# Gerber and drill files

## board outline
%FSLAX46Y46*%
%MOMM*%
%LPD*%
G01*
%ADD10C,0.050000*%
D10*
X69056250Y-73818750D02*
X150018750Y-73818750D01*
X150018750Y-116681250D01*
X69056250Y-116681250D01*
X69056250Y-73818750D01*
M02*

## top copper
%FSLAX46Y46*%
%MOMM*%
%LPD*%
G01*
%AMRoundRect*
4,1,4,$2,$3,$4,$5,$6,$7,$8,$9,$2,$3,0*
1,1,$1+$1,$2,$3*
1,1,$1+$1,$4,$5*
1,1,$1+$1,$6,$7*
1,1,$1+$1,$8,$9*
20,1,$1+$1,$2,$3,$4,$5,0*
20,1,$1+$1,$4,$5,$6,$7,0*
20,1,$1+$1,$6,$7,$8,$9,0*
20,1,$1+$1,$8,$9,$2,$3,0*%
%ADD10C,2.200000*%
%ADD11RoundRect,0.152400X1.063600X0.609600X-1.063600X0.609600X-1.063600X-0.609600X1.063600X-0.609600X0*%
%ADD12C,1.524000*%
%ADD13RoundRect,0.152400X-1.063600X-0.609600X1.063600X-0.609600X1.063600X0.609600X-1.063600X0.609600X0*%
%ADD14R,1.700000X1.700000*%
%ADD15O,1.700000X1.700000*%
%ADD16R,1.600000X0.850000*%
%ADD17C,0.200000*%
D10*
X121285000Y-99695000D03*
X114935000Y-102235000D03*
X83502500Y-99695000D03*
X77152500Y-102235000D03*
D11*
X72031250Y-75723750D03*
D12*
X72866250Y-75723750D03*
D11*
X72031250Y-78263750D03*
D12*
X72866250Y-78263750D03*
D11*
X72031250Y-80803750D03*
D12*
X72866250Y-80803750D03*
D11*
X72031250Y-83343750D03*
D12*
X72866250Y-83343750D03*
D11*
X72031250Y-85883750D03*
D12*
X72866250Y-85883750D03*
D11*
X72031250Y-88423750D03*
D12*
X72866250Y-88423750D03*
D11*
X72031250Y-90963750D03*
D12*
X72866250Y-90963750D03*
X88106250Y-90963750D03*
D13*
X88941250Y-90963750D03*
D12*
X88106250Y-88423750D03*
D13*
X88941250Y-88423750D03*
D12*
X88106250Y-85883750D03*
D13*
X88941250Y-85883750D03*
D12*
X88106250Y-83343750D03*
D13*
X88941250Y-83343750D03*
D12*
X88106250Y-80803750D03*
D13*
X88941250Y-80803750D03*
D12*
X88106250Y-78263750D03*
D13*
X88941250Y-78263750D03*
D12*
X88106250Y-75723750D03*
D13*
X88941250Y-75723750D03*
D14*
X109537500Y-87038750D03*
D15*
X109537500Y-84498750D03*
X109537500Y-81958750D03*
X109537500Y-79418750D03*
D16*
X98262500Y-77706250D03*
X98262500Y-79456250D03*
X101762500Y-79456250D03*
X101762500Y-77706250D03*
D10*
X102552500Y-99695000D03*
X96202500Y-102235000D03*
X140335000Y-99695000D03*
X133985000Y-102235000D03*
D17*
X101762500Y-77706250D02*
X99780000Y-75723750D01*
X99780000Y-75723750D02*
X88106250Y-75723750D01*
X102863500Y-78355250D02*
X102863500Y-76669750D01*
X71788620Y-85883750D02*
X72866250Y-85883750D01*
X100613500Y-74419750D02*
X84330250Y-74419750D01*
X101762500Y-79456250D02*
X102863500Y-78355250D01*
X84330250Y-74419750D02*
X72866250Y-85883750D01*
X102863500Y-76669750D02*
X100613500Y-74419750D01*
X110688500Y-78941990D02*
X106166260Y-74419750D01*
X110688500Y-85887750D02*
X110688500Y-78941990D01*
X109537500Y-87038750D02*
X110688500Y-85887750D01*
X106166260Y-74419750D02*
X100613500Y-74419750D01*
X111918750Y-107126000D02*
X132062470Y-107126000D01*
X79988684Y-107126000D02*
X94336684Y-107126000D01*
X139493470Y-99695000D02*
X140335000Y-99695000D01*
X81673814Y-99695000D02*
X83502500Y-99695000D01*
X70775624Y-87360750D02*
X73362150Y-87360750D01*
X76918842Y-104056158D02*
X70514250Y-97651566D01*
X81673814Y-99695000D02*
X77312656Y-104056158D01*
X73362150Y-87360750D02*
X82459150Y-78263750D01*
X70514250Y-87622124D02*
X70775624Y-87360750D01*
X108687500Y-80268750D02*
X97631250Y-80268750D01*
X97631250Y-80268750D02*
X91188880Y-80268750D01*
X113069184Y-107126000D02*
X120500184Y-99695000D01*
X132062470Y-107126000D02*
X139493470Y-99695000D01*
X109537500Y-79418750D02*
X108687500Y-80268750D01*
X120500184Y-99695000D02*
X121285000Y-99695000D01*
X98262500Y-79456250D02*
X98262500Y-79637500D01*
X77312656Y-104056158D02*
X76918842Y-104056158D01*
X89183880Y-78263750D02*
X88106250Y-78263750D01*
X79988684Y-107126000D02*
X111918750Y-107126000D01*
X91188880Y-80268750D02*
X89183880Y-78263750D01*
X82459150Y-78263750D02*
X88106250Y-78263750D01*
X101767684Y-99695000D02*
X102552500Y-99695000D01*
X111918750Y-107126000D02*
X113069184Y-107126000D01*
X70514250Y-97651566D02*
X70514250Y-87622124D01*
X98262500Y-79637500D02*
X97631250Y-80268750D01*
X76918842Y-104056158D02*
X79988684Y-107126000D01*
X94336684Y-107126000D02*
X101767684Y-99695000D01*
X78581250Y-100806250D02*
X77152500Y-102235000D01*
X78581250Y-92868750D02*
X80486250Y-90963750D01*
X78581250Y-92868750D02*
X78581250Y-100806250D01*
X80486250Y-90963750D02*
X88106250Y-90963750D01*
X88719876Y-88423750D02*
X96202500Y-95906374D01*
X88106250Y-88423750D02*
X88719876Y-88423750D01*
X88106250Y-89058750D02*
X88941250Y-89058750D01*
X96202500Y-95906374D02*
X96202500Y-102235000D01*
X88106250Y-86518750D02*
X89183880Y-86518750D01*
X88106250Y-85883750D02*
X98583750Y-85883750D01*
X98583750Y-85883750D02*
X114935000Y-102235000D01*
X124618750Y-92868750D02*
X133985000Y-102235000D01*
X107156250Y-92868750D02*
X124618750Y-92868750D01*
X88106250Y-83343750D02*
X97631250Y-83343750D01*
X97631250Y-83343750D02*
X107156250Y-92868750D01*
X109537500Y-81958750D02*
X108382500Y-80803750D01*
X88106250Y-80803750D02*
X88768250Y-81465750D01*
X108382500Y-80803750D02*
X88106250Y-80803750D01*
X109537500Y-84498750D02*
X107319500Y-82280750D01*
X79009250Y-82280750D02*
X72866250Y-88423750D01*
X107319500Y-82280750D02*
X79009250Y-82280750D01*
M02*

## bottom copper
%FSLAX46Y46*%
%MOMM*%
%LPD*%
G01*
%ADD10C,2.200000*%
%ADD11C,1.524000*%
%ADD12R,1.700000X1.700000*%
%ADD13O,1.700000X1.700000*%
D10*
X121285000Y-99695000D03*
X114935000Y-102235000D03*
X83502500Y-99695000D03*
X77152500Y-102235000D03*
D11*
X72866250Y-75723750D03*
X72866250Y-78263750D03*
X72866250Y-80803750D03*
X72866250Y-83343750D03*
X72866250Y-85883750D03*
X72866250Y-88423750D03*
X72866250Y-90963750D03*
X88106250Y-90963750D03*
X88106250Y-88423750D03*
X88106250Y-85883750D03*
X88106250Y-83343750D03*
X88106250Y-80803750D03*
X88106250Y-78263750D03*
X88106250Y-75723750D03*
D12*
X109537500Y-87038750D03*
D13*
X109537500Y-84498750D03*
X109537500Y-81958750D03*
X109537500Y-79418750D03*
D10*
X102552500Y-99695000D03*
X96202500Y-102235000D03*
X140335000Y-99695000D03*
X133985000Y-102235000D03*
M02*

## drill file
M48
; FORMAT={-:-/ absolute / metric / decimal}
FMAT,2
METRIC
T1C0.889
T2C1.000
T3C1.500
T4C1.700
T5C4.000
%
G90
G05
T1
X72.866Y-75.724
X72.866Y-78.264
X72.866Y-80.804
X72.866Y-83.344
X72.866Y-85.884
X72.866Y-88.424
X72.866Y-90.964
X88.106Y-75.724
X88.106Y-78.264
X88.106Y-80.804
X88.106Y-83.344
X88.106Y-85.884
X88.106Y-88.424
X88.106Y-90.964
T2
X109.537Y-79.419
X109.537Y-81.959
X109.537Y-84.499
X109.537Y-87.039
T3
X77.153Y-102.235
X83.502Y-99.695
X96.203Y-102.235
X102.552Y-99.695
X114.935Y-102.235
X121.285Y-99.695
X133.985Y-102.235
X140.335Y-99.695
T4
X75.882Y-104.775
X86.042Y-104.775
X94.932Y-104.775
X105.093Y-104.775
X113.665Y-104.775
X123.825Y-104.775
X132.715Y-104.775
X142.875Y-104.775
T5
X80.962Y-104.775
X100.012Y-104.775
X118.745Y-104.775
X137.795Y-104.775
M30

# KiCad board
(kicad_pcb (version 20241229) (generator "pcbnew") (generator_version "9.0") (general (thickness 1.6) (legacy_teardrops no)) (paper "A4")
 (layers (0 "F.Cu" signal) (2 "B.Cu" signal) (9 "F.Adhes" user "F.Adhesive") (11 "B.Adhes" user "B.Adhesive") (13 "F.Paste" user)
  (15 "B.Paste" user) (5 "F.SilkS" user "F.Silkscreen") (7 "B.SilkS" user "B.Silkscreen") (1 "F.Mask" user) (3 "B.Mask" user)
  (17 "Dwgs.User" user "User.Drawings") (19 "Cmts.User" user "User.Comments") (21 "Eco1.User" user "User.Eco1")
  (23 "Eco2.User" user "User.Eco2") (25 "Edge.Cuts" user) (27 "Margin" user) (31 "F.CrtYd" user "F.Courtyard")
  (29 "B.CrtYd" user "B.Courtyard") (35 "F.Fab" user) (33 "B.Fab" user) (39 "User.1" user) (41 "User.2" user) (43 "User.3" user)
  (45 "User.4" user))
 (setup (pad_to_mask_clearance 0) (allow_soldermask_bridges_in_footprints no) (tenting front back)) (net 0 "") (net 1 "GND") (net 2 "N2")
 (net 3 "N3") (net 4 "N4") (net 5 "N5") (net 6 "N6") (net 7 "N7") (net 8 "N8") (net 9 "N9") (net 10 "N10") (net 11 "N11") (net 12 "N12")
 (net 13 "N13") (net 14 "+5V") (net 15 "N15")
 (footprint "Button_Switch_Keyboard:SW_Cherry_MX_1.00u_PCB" (layer "F.Cu") (at 121.285 99.695)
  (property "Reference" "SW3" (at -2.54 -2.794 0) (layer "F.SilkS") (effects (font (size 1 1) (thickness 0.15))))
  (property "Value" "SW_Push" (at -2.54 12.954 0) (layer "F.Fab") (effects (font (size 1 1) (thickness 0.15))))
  (pad "" np_thru_hole circle (at -7.62 5.08) (size 1.7 1.7) (drill 1.7) (layers "*.Cu" "*.Mask"))
  (pad "" np_thru_hole circle (at -2.54 5.08) (size 4 4) (drill 4) (layers "*.Cu" "*.Mask"))
  (pad "" np_thru_hole circle (at 2.54 5.08) (size 1.7 1.7) (drill 1.7) (layers "*.Cu" "*.Mask"))
  (pad "1" thru_hole circle (at 0 0) (size 2.2 2.2) (drill 1.5) (layers "*.Cu" "*.Mask") (remove_unused_layers no) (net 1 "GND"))
  (pad "2" thru_hole circle (at -6.35 2.54) (size 2.2 2.2) (drill 1.5) (layers "*.Cu" "*.Mask") (remove_unused_layers no) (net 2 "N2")))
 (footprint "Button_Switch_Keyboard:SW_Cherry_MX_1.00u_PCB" (layer "F.Cu") (at 83.5025 99.695)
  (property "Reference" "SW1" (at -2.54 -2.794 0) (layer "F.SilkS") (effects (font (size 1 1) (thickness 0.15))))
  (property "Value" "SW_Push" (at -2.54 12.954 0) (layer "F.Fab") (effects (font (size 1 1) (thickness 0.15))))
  (pad "" np_thru_hole circle (at -7.62 5.08) (size 1.7 1.7) (drill 1.7) (layers "*.Cu" "*.Mask"))
  (pad "" np_thru_hole circle (at -2.54 5.08) (size 4 4) (drill 4) (layers "*.Cu" "*.Mask"))
  (pad "" np_thru_hole circle (at 2.54 5.08) (size 1.7 1.7) (drill 1.7) (layers "*.Cu" "*.Mask"))
  (pad "1" thru_hole circle (at 0 0) (size 2.2 2.2) (drill 1.5) (layers "*.Cu" "*.Mask") (remove_unused_layers no) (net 1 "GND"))
  (pad "2" thru_hole circle (at -6.35 2.54) (size 2.2 2.2) (drill 1.5) (layers "*.Cu" "*.Mask") (remove_unused_layers no) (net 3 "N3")))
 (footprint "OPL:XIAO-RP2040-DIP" (layer "F.Cu") (at 80.48625 83.34375)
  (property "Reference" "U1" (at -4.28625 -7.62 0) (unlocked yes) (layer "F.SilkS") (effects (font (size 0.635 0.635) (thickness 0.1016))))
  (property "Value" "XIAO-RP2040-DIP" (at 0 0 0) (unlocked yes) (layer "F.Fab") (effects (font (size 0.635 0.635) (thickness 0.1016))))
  (pad "1" smd roundrect (at -8.455 -7.62 180) (size 2.432 1.524) (layers "F.Cu" "F.Mask") (roundrect_rratio 0.1) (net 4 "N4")
   (thermal_bridge_angle 45))
  (pad "1" thru_hole circle (at -7.62 -7.62 180) (size 1.524 1.524) (drill 0.889) (layers "*.Cu" "*.Mask") (remove_unused_layers no)
   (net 4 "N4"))
  (pad "2" smd roundrect (at -8.455 -5.08 180) (size 2.432 1.524) (layers "F.Cu" "F.Mask") (roundrect_rratio 0.1) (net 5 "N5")
   (thermal_bridge_angle 45))
  (pad "2" thru_hole circle (at -7.62 -5.08 180) (size 1.524 1.524) (drill 0.889) (layers "*.Cu" "*.Mask") (remove_unused_layers no)
   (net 5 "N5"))
  (pad "3" smd roundrect (at -8.455 -2.54 180) (size 2.432 1.524) (layers "F.Cu" "F.Mask") (roundrect_rratio 0.1) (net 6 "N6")
   (thermal_bridge_angle 45))
  (pad "3" thru_hole circle (at -7.62 -2.54 180) (size 1.524 1.524) (drill 0.889) (layers "*.Cu" "*.Mask") (remove_unused_layers no)
   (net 6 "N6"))
  (pad "4" smd roundrect (at -8.455 0 180) (size 2.432 1.524) (layers "F.Cu" "F.Mask") (roundrect_rratio 0.1) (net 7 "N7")
   (thermal_bridge_angle 45))
  (pad "4" thru_hole circle (at -7.62 0 180) (size 1.524 1.524) (drill 0.889) (layers "*.Cu" "*.Mask") (remove_unused_layers no)
   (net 7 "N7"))
  (pad "5" smd roundrect (at -8.455 2.54 180) (size 2.432 1.524) (layers "F.Cu" "F.Mask") (roundrect_rratio 0.1) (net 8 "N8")
   (thermal_bridge_angle 45))
  (pad "5" thru_hole circle (at -7.62 2.54 180) (size 1.524 1.524) (drill 0.889) (layers "*.Cu" "*.Mask") (remove_unused_layers no)
   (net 8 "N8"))
  (pad "6" smd roundrect (at -8.455 5.08 180) (size 2.432 1.524) (layers "F.Cu" "F.Mask") (roundrect_rratio 0.1) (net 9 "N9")
   (thermal_bridge_angle 45))
  (pad "6" thru_hole circle (at -7.62 5.08 180) (size 1.524 1.524) (drill 0.889) (layers "*.Cu" "*.Mask") (remove_unused_layers no)
   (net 9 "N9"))
  (pad "7" smd roundrect (at -8.455 7.62 180) (size 2.432 1.524) (layers "F.Cu" "F.Mask") (roundrect_rratio 0.1) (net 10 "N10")
   (thermal_bridge_angle 45))
  (pad "7" thru_hole circle (at -7.62 7.62 180) (size 1.524 1.524) (drill 0.889) (layers "*.Cu" "*.Mask") (remove_unused_layers no)
   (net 10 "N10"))
  (pad "8" thru_hole circle (at 7.62 7.62) (size 1.524 1.524) (drill 0.889) (layers "*.Cu" "*.Mask") (remove_unused_layers no) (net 3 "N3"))
  (pad "8" smd roundrect (at 8.455 7.62) (size 2.432 1.524) (layers "F.Cu" "F.Mask") (roundrect_rratio 0.1) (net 3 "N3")
   (thermal_bridge_angle 45))
  (pad "9" thru_hole circle (at 7.62 5.08) (size 1.524 1.524) (drill 0.889) (layers "*.Cu" "*.Mask") (remove_unused_layers no)
   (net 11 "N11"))
  (pad "9" smd roundrect (at 8.455 5.08) (size 2.432 1.524) (layers "F.Cu" "F.Mask") (roundrect_rratio 0.1) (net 11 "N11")
   (thermal_bridge_angle 45))
  (pad "10" thru_hole circle (at 7.62 2.54) (size 1.524 1.524) (drill 0.889) (layers "*.Cu" "*.Mask") (remove_unused_layers no) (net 2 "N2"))
  (pad "10" smd roundrect (at 8.455 2.54) (size 2.432 1.524) (layers "F.Cu" "F.Mask") (roundrect_rratio 0.1) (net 2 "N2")
   (thermal_bridge_angle 45))
  (pad "11" thru_hole circle (at 7.62 0) (size 1.524 1.524) (drill 0.889) (layers "*.Cu" "*.Mask") (remove_unused_layers no) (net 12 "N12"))
  (pad "11" smd roundrect (at 8.455 0) (size 2.432 1.524) (layers "F.Cu" "F.Mask") (roundrect_rratio 0.1) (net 12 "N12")
   (thermal_bridge_angle 45))
  (pad "12" thru_hole circle (at 7.62 -2.54) (size 1.524 1.524) (drill 0.889) (layers "*.Cu" "*.Mask") (remove_unused_layers no)
   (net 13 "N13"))
  (pad "12" smd roundrect (at 8.455 -2.54) (size 2.432 1.524) (layers "F.Cu" "F.Mask") (roundrect_rratio 0.1) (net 13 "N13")
   (thermal_bridge_angle 45))
  (pad "13" thru_hole circle (at 7.62 -5.08) (size 1.524 1.524) (drill 0.889) (layers "*.Cu" "*.Mask") (remove_unused_layers no)
   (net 1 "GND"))
  (pad "13" smd roundrect (at 8.455 -5.08) (size 2.432 1.524) (layers "F.Cu" "F.Mask") (roundrect_rratio 0.1) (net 1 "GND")
   (thermal_bridge_angle 45))
  (pad "14" thru_hole circle (at 7.62 -7.62) (size 1.524 1.524) (drill 0.889) (layers "*.Cu" "*.Mask") (remove_unused_layers no)
   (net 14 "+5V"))
  (pad "14" smd roundrect (at 8.455 -7.62) (size 2.432 1.524) (layers "F.Cu" "F.Mask") (roundrect_rratio 0.1) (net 14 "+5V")
   (thermal_bridge_angle 45)))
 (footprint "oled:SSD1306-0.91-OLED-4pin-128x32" (layer "F.Cu") (at 146.0375 89.22875 180)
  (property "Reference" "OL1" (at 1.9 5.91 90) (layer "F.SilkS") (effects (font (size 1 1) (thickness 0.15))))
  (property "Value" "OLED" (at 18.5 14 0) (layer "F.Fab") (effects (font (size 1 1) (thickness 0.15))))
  (pad "1" thru_hole rect (at 36.5 2.19 180) (size 1.7 1.7) (drill 1) (layers "*.Cu" "*.Mask") (remove_unused_layers no) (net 8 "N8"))
  (pad "2" thru_hole oval (at 36.5 4.73 180) (size 1.7 1.7) (drill 1) (layers "*.Cu" "*.Mask") (remove_unused_layers no) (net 9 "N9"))
  (pad "3" thru_hole oval (at 36.5 7.27 180) (size 1.7 1.7) (drill 1) (layers "*.Cu" "*.Mask") (remove_unused_layers no) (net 13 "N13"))
  (pad "4" thru_hole oval (at 36.5 9.81 180) (size 1.7 1.7) (drill 1) (layers "*.Cu" "*.Mask") (remove_unused_layers no) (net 1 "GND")))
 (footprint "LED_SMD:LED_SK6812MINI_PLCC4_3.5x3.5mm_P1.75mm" (layer "F.Cu") (at 100.0125 78.58125)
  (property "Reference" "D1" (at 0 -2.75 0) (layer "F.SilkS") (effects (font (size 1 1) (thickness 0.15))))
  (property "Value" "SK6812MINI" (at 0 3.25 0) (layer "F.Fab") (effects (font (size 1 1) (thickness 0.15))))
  (pad "1" smd rect (at -1.75 -0.875) (size 1.6 0.85) (layers "F.Cu" "F.Mask" "F.Paste") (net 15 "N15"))
  (pad "2" smd rect (at -1.75 0.875) (size 1.6 0.85) (layers "F.Cu" "F.Mask" "F.Paste") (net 1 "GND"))
  (pad "3" smd rect (at 1.75 0.875) (size 1.6 0.85) (layers "F.Cu" "F.Mask" "F.Paste") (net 8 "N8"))
  (pad "4" smd rect (at 1.75 -0.875) (size 1.6 0.85) (layers "F.Cu" "F.Mask" "F.Paste") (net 14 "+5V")))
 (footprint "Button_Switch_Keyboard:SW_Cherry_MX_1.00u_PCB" (layer "F.Cu") (at 102.5525 99.695)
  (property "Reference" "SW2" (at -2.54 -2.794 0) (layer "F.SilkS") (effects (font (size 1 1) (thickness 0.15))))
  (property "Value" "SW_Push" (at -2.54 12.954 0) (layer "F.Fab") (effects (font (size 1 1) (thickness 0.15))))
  (pad "" np_thru_hole circle (at -7.62 5.08) (size 1.7 1.7) (drill 1.7) (layers "*.Cu" "*.Mask"))
  (pad "" np_thru_hole circle (at -2.54 5.08) (size 4 4) (drill 4) (layers "*.Cu" "*.Mask"))
  (pad "" np_thru_hole circle (at 2.54 5.08) (size 1.7 1.7) (drill 1.7) (layers "*.Cu" "*.Mask"))
  (pad "1" thru_hole circle (at 0 0) (size 2.2 2.2) (drill 1.5) (layers "*.Cu" "*.Mask") (remove_unused_layers no) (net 1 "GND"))
  (pad "2" thru_hole circle (at -6.35 2.54) (size 2.2 2.2) (drill 1.5) (layers "*.Cu" "*.Mask") (remove_unused_layers no) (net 11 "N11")))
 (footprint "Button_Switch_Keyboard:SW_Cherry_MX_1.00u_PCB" (layer "F.Cu") (at 140.335 99.695)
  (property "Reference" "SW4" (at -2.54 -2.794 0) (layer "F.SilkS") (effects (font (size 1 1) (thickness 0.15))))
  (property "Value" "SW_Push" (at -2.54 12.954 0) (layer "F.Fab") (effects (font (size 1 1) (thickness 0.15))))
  (pad "" np_thru_hole circle (at -7.62 5.08) (size 1.7 1.7) (drill 1.7) (layers "*.Cu" "*.Mask"))
  (pad "" np_thru_hole circle (at -2.54 5.08) (size 4 4) (drill 4) (layers "*.Cu" "*.Mask"))
  (pad "" np_thru_hole circle (at 2.54 5.08) (size 1.7 1.7) (drill 1.7) (layers "*.Cu" "*.Mask"))
  (pad "1" thru_hole circle (at 0 0) (size 2.2 2.2) (drill 1.5) (layers "*.Cu" "*.Mask") (remove_unused_layers no) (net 1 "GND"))
  (pad "2" thru_hole circle (at -6.35 2.54) (size 2.2 2.2) (drill 1.5) (layers "*.Cu" "*.Mask") (remove_unused_layers no) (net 12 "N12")))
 (gr_rect (start 69.05625 73.81875) (end 150.01875 116.68125) (stroke (width 0.05) (type default)) (fill no) (layer "Edge.Cuts"))
 (segment (start 101.7625 77.70625) (end 99.78 75.72375) (width 0.2) (layer "F.Cu") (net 14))
 (segment (start 99.78 75.72375) (end 88.10625 75.72375) (width 0.2) (layer "F.Cu") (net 14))
 (segment (start 102.8635 78.35525) (end 102.8635 76.66975) (width 0.2) (layer "F.Cu") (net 8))
 (segment (start 71.78862 85.88375) (end 72.86625 85.88375) (width 0.2) (layer "F.Cu") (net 8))
 (segment (start 100.6135 74.41975) (end 84.33025 74.41975) (width 0.2) (layer "F.Cu") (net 8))
 (segment (start 101.7625 79.45625) (end 102.8635 78.35525) (width 0.2) (layer "F.Cu") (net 8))
 (segment (start 84.33025 74.41975) (end 72.86625 85.88375) (width 0.2) (layer "F.Cu") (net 8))
 (segment (start 102.8635 76.66975) (end 100.6135 74.41975) (width 0.2) (layer "F.Cu") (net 8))
 (segment (start 110.6885 78.94199) (end 106.16626 74.41975) (width 0.2) (layer "F.Cu") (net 8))
 (segment (start 110.6885 85.88775) (end 110.6885 78.94199) (width 0.2) (layer "F.Cu") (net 8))
 (segment (start 109.5375 87.03875) (end 110.6885 85.88775) (width 0.2) (layer "F.Cu") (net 8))
 (segment (start 106.16626 74.41975) (end 100.6135 74.41975) (width 0.2) (layer "F.Cu") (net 8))
 (segment (start 111.91875 107.126) (end 132.06247 107.126) (width 0.2) (layer "F.Cu") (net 1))
 (segment (start 79.988684 107.126) (end 94.336684 107.126) (width 0.2) (layer "F.Cu") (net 1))
 (segment (start 139.49347 99.695) (end 140.335 99.695) (width 0.2) (layer "F.Cu") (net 1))
 (segment (start 81.673814 99.695) (end 83.5025 99.695) (width 0.2) (layer "F.Cu") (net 1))
 (segment (start 70.775624 87.36075) (end 73.36215 87.36075) (width 0.2) (layer "F.Cu") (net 1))
 (segment (start 76.918842 104.056158) (end 70.51425 97.651566) (width 0.2) (layer "F.Cu") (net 1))
 (segment (start 81.673814 99.695) (end 77.312656 104.056158) (width 0.2) (layer "F.Cu") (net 1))
 (segment (start 73.36215 87.36075) (end 82.45915 78.26375) (width 0.2) (layer "F.Cu") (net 1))
 (segment (start 70.51425 87.622124) (end 70.775624 87.36075) (width 0.2) (layer "F.Cu") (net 1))
 (segment (start 108.6875 80.26875) (end 97.63125 80.26875) (width 0.2) (layer "F.Cu") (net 1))
 (segment (start 97.63125 80.26875) (end 91.18888 80.26875) (width 0.2) (layer "F.Cu") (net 1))
 (segment (start 113.069184 107.126) (end 120.500184 99.695) (width 0.2) (layer "F.Cu") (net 1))
 (segment (start 132.06247 107.126) (end 139.49347 99.695) (width 0.2) (layer "F.Cu") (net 1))
 (segment (start 109.5375 79.41875) (end 108.6875 80.26875) (width 0.2) (layer "F.Cu") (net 1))
 (segment (start 120.500184 99.695) (end 121.285 99.695) (width 0.2) (layer "F.Cu") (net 1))
 (segment (start 98.2625 79.45625) (end 98.2625 79.6375) (width 0.2) (layer "F.Cu") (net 1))
 (segment (start 77.312656 104.056158) (end 76.918842 104.056158) (width 0.2) (layer "F.Cu") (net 1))
 (segment (start 89.18388 78.26375) (end 88.10625 78.26375) (width 0.2) (layer "F.Cu") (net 1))
 (segment (start 79.988684 107.126) (end 111.91875 107.126) (width 0.2) (layer "F.Cu") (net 1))
 (segment (start 91.18888 80.26875) (end 89.18388 78.26375) (width 0.2) (layer "F.Cu") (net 1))
 (segment (start 82.45915 78.26375) (end 88.10625 78.26375) (width 0.2) (layer "F.Cu") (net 1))
 (segment (start 101.767684 99.695) (end 102.5525 99.695) (width 0.2) (layer "F.Cu") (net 1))
 (segment (start 111.91875 107.126) (end 113.069184 107.126) (width 0.2) (layer "F.Cu") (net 1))
 (segment (start 70.51425 97.651566) (end 70.51425 87.622124) (width 0.2) (layer "F.Cu") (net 1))
 (segment (start 98.2625 79.6375) (end 97.63125 80.26875) (width 0.2) (layer "F.Cu") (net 1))
 (segment (start 76.918842 104.056158) (end 79.988684 107.126) (width 0.2) (layer "F.Cu") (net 1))
 (segment (start 94.336684 107.126) (end 101.767684 99.695) (width 0.2) (layer "F.Cu") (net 1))
 (segment (start 78.58125 100.80625) (end 77.1525 102.235) (width 0.2) (layer "F.Cu") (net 3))
 (segment (start 78.58125 92.86875) (end 80.48625 90.96375) (width 0.2) (layer "F.Cu") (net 3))
 (segment (start 78.58125 92.86875) (end 78.58125 100.80625) (width 0.2) (layer "F.Cu") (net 3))
 (segment (start 80.48625 90.96375) (end 88.10625 90.96375) (width 0.2) (layer "F.Cu") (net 3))
 (segment (start 88.719876 88.42375) (end 96.2025 95.906374) (width 0.2) (layer "F.Cu") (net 11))
 (segment (start 88.10625 88.42375) (end 88.719876 88.42375) (width 0.2) (layer "F.Cu") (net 11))
 (segment (start 88.10625 89.05875) (end 88.94125 89.05875) (width 0.2) (layer "F.Cu") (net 11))
 (segment (start 96.2025 95.906374) (end 96.2025 102.235) (width 0.2) (layer "F.Cu") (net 11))
 (segment (start 88.10625 86.51875) (end 89.18388 86.51875) (width 0.2) (layer "F.Cu") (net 2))
 (segment (start 88.10625 85.88375) (end 98.58375 85.88375) (width 0.2) (layer "F.Cu") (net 2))
 (segment (start 98.58375 85.88375) (end 114.935 102.235) (width 0.2) (layer "F.Cu") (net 2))
 (segment (start 124.61875 92.86875) (end 133.985 102.235) (width 0.2) (layer "F.Cu") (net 12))
 (segment (start 107.15625 92.86875) (end 124.61875 92.86875) (width 0.2) (layer "F.Cu") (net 12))
 (segment (start 88.10625 83.34375) (end 97.63125 83.34375) (width 0.2) (layer "F.Cu") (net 12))
 (segment (start 97.63125 83.34375) (end 107.15625 92.86875) (width 0.2) (layer "F.Cu") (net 12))
 (segment (start 109.5375 81.95875) (end 108.3825 80.80375) (width 0.2) (layer "F.Cu") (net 13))
 (segment (start 88.10625 80.80375) (end 88.76825 81.46575) (width 0.2) (layer "F.Cu") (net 13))
 (segment (start 108.3825 80.80375) (end 88.10625 80.80375) (width 0.2) (layer "F.Cu") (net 13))
 (segment (start 109.5375 84.49875) (end 107.3195 82.28075) (width 0.2) (layer "F.Cu") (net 9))
 (segment (start 79.00925 82.28075) (end 72.86625 88.42375) (width 0.2) (layer "F.Cu") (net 9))
 (segment (start 107.3195 82.28075) (end 79.00925 82.28075) (width 0.2) (layer "F.Cu") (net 9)))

